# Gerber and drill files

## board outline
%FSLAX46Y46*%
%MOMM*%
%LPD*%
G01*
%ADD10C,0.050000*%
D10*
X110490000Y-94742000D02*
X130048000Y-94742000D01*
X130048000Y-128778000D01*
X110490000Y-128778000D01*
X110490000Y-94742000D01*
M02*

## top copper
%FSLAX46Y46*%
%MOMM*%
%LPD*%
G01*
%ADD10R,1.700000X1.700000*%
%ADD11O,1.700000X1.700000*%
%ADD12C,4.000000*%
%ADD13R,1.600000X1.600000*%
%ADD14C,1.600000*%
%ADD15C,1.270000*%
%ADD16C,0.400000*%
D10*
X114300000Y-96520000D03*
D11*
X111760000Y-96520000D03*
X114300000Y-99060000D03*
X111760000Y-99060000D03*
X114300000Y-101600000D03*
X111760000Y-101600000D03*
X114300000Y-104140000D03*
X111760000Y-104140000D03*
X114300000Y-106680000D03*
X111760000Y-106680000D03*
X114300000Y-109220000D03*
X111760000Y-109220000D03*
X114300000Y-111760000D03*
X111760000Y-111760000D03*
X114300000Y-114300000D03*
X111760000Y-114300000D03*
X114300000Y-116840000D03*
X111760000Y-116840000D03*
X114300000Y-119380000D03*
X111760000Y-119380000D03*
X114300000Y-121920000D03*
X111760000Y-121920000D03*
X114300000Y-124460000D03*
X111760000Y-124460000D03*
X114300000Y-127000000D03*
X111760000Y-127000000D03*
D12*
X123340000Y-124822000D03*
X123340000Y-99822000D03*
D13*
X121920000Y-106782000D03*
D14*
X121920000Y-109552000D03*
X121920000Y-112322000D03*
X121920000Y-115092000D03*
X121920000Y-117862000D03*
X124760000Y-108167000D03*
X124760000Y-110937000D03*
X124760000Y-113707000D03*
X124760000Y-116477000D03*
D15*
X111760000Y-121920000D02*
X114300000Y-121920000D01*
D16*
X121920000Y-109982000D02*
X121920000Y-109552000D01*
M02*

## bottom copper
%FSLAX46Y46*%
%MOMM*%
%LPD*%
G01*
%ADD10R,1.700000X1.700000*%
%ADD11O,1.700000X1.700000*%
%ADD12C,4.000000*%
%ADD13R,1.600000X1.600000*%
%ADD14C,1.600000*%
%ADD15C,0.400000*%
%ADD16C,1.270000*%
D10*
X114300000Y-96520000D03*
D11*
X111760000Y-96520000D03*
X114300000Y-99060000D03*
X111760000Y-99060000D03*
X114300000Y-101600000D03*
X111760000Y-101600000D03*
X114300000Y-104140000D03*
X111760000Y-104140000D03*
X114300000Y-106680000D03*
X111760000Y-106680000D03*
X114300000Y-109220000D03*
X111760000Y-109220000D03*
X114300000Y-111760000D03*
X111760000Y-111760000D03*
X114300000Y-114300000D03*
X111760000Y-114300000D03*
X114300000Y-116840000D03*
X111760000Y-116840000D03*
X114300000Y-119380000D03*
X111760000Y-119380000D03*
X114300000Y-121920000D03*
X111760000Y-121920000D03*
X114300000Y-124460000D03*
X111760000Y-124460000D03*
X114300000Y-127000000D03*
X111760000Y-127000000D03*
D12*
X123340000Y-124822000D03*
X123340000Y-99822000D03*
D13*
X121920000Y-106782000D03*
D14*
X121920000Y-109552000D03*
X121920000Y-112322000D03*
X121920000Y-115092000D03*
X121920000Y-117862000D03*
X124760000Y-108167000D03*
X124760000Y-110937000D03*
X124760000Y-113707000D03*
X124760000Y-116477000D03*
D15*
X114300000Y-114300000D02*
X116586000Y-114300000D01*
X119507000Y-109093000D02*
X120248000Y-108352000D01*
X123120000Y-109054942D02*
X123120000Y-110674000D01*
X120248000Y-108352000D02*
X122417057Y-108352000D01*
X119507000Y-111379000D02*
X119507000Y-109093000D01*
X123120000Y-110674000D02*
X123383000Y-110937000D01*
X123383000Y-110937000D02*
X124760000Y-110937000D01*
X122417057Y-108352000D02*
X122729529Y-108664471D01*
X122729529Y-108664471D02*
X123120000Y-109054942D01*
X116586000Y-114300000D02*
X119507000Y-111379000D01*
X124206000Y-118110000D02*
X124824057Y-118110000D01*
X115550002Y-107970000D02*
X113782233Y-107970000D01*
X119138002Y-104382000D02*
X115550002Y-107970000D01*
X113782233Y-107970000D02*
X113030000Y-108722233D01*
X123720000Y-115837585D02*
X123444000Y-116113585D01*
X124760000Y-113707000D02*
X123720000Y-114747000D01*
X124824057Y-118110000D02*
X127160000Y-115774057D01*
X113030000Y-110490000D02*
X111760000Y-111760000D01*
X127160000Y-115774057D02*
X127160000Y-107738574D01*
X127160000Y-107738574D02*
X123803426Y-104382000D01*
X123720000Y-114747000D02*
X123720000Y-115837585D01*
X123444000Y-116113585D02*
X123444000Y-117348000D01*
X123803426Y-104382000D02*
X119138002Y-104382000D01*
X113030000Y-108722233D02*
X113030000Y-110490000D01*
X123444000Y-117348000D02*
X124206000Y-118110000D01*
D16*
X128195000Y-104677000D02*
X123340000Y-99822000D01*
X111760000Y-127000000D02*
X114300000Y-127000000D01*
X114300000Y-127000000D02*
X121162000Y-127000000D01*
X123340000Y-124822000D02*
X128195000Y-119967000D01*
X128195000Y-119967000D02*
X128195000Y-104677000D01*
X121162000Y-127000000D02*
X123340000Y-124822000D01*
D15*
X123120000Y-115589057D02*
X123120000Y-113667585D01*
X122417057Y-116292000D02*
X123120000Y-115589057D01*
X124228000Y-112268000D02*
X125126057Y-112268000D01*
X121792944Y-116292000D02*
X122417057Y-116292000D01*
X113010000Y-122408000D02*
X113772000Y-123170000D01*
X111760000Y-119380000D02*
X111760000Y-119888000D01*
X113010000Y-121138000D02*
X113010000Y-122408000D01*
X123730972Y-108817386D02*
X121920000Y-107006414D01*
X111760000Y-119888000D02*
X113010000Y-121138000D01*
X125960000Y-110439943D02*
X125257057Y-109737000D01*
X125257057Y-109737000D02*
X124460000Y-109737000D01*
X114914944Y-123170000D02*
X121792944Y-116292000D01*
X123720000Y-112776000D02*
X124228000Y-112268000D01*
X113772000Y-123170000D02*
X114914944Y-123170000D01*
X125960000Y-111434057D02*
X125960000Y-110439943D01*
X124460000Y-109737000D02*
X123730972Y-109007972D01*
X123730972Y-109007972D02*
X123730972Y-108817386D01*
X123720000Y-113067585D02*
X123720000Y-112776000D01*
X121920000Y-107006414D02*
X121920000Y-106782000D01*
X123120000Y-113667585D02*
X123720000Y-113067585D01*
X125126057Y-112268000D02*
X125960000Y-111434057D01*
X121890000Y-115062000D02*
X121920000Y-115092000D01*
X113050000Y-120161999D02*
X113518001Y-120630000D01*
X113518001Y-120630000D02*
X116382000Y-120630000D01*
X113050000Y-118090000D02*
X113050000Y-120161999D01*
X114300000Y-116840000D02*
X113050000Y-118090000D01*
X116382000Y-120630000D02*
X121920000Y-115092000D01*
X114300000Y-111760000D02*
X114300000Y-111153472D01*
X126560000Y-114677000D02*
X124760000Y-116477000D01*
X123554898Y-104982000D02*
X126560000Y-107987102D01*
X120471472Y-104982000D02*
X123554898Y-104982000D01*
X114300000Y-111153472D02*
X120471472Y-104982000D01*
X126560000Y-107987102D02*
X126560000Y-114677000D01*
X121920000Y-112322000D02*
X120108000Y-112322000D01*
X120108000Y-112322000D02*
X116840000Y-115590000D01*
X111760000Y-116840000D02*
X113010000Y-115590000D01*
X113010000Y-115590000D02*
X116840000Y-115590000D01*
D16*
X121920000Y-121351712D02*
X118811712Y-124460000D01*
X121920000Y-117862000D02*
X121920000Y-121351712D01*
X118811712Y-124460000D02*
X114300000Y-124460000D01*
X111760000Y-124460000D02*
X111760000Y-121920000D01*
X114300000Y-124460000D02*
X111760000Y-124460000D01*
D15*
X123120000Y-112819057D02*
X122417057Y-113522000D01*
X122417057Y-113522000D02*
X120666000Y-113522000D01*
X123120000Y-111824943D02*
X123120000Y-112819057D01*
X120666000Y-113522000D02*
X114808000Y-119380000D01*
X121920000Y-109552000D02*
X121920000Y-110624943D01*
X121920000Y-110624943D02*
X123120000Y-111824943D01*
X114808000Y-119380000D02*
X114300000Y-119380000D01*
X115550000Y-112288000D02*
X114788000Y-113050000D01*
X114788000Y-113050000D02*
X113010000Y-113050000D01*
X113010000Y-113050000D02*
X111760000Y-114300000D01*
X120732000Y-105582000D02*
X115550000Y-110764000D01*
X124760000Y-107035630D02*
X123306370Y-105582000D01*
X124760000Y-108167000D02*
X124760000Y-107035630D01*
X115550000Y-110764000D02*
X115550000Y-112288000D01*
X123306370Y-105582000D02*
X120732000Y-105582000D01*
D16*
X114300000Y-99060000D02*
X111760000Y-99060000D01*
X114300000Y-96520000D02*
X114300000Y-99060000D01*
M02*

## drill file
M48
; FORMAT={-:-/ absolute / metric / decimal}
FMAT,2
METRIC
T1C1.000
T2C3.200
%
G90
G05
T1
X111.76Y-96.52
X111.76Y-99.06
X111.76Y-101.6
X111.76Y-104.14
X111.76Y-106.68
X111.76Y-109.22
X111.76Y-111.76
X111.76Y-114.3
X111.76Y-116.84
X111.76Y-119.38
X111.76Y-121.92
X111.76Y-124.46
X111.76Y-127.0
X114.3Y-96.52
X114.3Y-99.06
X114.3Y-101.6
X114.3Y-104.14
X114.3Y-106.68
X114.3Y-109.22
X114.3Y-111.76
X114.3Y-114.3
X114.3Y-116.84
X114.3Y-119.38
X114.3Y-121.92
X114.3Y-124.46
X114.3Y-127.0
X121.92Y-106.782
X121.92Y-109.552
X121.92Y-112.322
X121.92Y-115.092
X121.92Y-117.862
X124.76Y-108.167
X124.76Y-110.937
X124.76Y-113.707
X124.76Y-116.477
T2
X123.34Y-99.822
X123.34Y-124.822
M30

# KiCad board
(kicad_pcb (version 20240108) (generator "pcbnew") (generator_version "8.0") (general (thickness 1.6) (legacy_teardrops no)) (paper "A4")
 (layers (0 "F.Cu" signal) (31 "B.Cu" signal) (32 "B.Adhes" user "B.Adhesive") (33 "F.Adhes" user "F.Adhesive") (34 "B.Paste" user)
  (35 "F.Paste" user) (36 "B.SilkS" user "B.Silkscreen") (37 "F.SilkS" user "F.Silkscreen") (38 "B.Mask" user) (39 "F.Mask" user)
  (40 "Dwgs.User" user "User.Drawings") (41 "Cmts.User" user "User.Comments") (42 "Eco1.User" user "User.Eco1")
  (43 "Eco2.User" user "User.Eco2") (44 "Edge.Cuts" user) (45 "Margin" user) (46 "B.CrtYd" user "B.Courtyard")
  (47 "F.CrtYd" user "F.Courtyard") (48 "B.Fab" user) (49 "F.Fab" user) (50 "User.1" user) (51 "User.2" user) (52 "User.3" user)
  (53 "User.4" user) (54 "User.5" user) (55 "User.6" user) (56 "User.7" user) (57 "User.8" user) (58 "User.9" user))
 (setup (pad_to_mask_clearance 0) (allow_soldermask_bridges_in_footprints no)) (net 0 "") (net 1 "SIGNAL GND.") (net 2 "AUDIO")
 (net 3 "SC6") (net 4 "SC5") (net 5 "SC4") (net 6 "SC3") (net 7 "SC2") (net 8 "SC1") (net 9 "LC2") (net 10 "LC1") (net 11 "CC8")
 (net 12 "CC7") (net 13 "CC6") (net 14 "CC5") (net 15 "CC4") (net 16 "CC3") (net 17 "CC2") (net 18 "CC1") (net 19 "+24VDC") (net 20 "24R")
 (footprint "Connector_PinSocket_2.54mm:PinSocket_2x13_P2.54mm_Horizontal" (layer "F.Cu") (at 114.3 96.52)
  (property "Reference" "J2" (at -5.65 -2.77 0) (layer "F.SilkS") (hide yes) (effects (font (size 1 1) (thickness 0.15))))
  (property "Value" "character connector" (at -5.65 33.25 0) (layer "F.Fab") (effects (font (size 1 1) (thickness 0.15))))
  (pad "1" thru_hole rect (at 0 0) (size 1.7 1.7) (drill 1) (layers "*.Cu" "*.Mask") (remove_unused_layers no) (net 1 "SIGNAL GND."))
  (pad "2" thru_hole oval (at -2.54 0) (size 1.7 1.7) (drill 1) (layers "*.Cu" "*.Mask") (remove_unused_layers no) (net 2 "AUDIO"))
  (pad "3" thru_hole oval (at 0 2.54) (size 1.7 1.7) (drill 1) (layers "*.Cu" "*.Mask") (remove_unused_layers no) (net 1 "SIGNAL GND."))
  (pad "4" thru_hole oval (at -2.54 2.54) (size 1.7 1.7) (drill 1) (layers "*.Cu" "*.Mask") (remove_unused_layers no) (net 1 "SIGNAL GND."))
  (pad "5" thru_hole oval (at 0 5.08) (size 1.7 1.7) (drill 1) (layers "*.Cu" "*.Mask") (remove_unused_layers no) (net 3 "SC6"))
  (pad "6" thru_hole oval (at -2.54 5.08) (size 1.7 1.7) (drill 1) (layers "*.Cu" "*.Mask") (remove_unused_layers no) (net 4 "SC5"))
  (pad "7" thru_hole oval (at 0 7.62) (size 1.7 1.7) (drill 1) (layers "*.Cu" "*.Mask") (remove_unused_layers no) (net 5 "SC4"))
  (pad "8" thru_hole oval (at -2.54 7.62) (size 1.7 1.7) (drill 1) (layers "*.Cu" "*.Mask") (remove_unused_layers no) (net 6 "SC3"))
  (pad "9" thru_hole oval (at 0 10.16) (size 1.7 1.7) (drill 1) (layers "*.Cu" "*.Mask") (remove_unused_layers no) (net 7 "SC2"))
  (pad "10" thru_hole oval (at -2.54 10.16) (size 1.7 1.7) (drill 1) (layers "*.Cu" "*.Mask") (remove_unused_layers no) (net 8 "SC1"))
  (pad "11" thru_hole oval (at 0 12.7) (size 1.7 1.7) (drill 1) (layers "*.Cu" "*.Mask") (remove_unused_layers no) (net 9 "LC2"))
  (pad "12" thru_hole oval (at -2.54 12.7) (size 1.7 1.7) (drill 1) (layers "*.Cu" "*.Mask") (remove_unused_layers no) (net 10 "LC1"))
  (pad "13" thru_hole oval (at 0 15.24) (size 1.7 1.7) (drill 1) (layers "*.Cu" "*.Mask") (remove_unused_layers no) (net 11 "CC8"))
  (pad "14" thru_hole oval (at -2.54 15.24) (size 1.7 1.7) (drill 1) (layers "*.Cu" "*.Mask") (remove_unused_layers no) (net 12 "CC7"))
  (pad "15" thru_hole oval (at 0 17.78) (size 1.7 1.7) (drill 1) (layers "*.Cu" "*.Mask") (remove_unused_layers no) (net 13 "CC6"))
  (pad "16" thru_hole oval (at -2.54 17.78) (size 1.7 1.7) (drill 1) (layers "*.Cu" "*.Mask") (remove_unused_layers no) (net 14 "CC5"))
  (pad "17" thru_hole oval (at 0 20.32) (size 1.7 1.7) (drill 1) (layers "*.Cu" "*.Mask") (remove_unused_layers no) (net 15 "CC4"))
  (pad "18" thru_hole oval (at -2.54 20.32) (size 1.7 1.7) (drill 1) (layers "*.Cu" "*.Mask") (remove_unused_layers no) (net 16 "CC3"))
  (pad "19" thru_hole oval (at 0 22.86) (size 1.7 1.7) (drill 1) (layers "*.Cu" "*.Mask") (remove_unused_layers no) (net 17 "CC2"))
  (pad "20" thru_hole oval (at -2.54 22.86) (size 1.7 1.7) (drill 1) (layers "*.Cu" "*.Mask") (remove_unused_layers no) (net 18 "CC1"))
  (pad "21" thru_hole oval (at 0 25.4) (size 1.7 1.7) (drill 1) (layers "*.Cu" "*.Mask") (remove_unused_layers no) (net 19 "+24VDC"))
  (pad "22" thru_hole oval (at -2.54 25.4) (size 1.7 1.7) (drill 1) (layers "*.Cu" "*.Mask") (remove_unused_layers no) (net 19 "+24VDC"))
  (pad "23" thru_hole oval (at 0 27.94) (size 1.7 1.7) (drill 1) (layers "*.Cu" "*.Mask") (remove_unused_layers no) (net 19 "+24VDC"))
  (pad "24" thru_hole oval (at -2.54 27.94) (size 1.7 1.7) (drill 1) (layers "*.Cu" "*.Mask") (remove_unused_layers no) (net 19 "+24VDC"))
  (pad "25" thru_hole oval (at 0 30.48) (size 1.7 1.7) (drill 1) (layers "*.Cu" "*.Mask") (remove_unused_layers no) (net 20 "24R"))
  (pad "26" thru_hole oval (at -2.54 30.48) (size 1.7 1.7) (drill 1) (layers "*.Cu" "*.Mask") (remove_unused_layers no) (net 20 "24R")))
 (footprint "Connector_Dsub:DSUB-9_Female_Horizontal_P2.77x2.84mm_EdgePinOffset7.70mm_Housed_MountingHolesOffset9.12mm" (layer "F.Cu")
  (at 121.92 106.782 90)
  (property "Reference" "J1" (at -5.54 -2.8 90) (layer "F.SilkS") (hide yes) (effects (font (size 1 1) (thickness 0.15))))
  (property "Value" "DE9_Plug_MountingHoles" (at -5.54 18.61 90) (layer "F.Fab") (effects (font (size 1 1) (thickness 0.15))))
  (pad "0" thru_hole circle (at -18.04 1.42 90) (size 4 4) (drill 3.2) (layers "*.Cu" "*.Mask") (remove_unused_layers no) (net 20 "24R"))
  (pad "0" thru_hole circle (at 6.96 1.42 90) (size 4 4) (drill 3.2) (layers "*.Cu" "*.Mask") (remove_unused_layers no) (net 20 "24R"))
  (pad "1" thru_hole rect (at 0 0 90) (size 1.6 1.6) (drill 1) (layers "*.Cu" "*.Mask") (remove_unused_layers no) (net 18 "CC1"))
  (pad "2" thru_hole circle (at -2.77 0 90) (size 1.6 1.6) (drill 1) (layers "*.Cu" "*.Mask") (remove_unused_layers no) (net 17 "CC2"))
  (pad "3" thru_hole circle (at -5.54 0 90) (size 1.6 1.6) (drill 1) (layers "*.Cu" "*.Mask") (remove_unused_layers no) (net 16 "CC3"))
  (pad "4" thru_hole circle (at -8.31 0 90) (size 1.6 1.6) (drill 1) (layers "*.Cu" "*.Mask") (remove_unused_layers no) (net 15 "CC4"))
  (pad "5" thru_hole circle (at -11.08 0 90) (size 1.6 1.6) (drill 1) (layers "*.Cu" "*.Mask") (remove_unused_layers no) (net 19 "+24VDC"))
  (pad "6" thru_hole circle (at -1.385 2.84 90) (size 1.6 1.6) (drill 1) (layers "*.Cu" "*.Mask") (remove_unused_layers no) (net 14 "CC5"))
  (pad "7" thru_hole circle (at -4.155 2.84 90) (size 1.6 1.6) (drill 1) (layers "*.Cu" "*.Mask") (remove_unused_layers no) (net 13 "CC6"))
  (pad "8" thru_hole circle (at -6.925 2.84 90) (size 1.6 1.6) (drill 1) (layers "*.Cu" "*.Mask") (remove_unused_layers no) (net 12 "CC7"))
  (pad "9" thru_hole circle (at -9.695 2.84 90) (size 1.6 1.6) (drill 1) (layers "*.Cu" "*.Mask") (remove_unused_layers no) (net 11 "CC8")))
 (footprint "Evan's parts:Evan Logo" (layer "B.Cu") (at 127.254 97.536 -90)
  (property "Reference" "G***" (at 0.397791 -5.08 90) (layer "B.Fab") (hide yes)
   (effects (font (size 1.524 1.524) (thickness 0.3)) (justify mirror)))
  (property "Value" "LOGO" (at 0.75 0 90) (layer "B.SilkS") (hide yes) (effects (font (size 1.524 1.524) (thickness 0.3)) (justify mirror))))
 (gr_rect (start 110.49 94.742) (end 130.048 128.778) (stroke (width 0.05) (type default)) (fill none) (layer "Edge.Cuts"))
 (segment (start 114.3 114.3) (end 116.586 114.3) (width 0.4) (layer "B.Cu") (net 13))
 (segment (start 119.507 109.093) (end 120.248 108.352) (width 0.4) (layer "B.Cu") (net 13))
 (segment (start 123.12 109.054942) (end 123.12 110.674) (width 0.4) (layer "B.Cu") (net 13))
 (segment (start 120.248 108.352) (end 122.417057 108.352) (width 0.4) (layer "B.Cu") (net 13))
 (segment (start 119.507 111.379) (end 119.507 109.093) (width 0.4) (layer "B.Cu") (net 13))
 (segment (start 123.12 110.674) (end 123.383 110.937) (width 0.4) (layer "B.Cu") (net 13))
 (segment (start 123.383 110.937) (end 124.76 110.937) (width 0.4) (layer "B.Cu") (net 13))
 (segment (start 122.417057 108.352) (end 122.729529 108.664471) (width 0.4) (layer "B.Cu") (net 13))
 (segment (start 122.729529 108.664471) (end 123.12 109.054942) (width 0.4) (layer "B.Cu") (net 13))
 (segment (start 116.586 114.3) (end 119.507 111.379) (width 0.4) (layer "B.Cu") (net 13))
 (segment (start 124.206 118.11) (end 124.824057 118.11) (width 0.4) (layer "B.Cu") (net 12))
 (segment (start 115.550002 107.97) (end 113.782233 107.97) (width 0.4) (layer "B.Cu") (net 12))
 (segment (start 119.138002 104.382) (end 115.550002 107.97) (width 0.4) (layer "B.Cu") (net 12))
 (segment (start 113.782233 107.97) (end 113.03 108.722233) (width 0.4) (layer "B.Cu") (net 12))
 (segment (start 123.72 115.837585) (end 123.444 116.113585) (width 0.4) (layer "B.Cu") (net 12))
 (segment (start 124.76 113.707) (end 123.72 114.747) (width 0.4) (layer "B.Cu") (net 12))
 (segment (start 124.824057 118.11) (end 127.16 115.774057) (width 0.4) (layer "B.Cu") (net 12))
 (segment (start 113.03 110.49) (end 111.76 111.76) (width 0.4) (layer "B.Cu") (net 12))
 (segment (start 127.16 115.774057) (end 127.16 107.738574) (width 0.4) (layer "B.Cu") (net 12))
 (segment (start 127.16 107.738574) (end 123.803426 104.382) (width 0.4) (layer "B.Cu") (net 12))
 (segment (start 123.72 114.747) (end 123.72 115.837585) (width 0.4) (layer "B.Cu") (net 12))
 (segment (start 123.444 116.113585) (end 123.444 117.348) (width 0.4) (layer "B.Cu") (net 12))
 (segment (start 123.803426 104.382) (end 119.138002 104.382) (width 0.4) (layer "B.Cu") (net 12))
 (segment (start 113.03 108.722233) (end 113.03 110.49) (width 0.4) (layer "B.Cu") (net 12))
 (segment (start 123.444 117.348) (end 124.206 118.11) (width 0.4) (layer "B.Cu") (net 12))
 (segment (start 128.195 104.677) (end 123.34 99.822) (width 1.27) (layer "B.Cu") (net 20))
 (segment (start 111.76 127) (end 114.3 127) (width 1.27) (layer "B.Cu") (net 20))
 (segment (start 114.3 127) (end 121.162 127) (width 1.27) (layer "B.Cu") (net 20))
 (segment (start 123.34 124.822) (end 128.195 119.967) (width 1.27) (layer "B.Cu") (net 20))
 (segment (start 128.195 119.967) (end 128.195 104.677) (width 1.27) (layer "B.Cu") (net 20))
 (segment (start 121.162 127) (end 123.34 124.822) (width 1.27) (layer "B.Cu") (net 20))
 (segment (start 123.12 115.589057) (end 123.12 113.667585) (width 0.4) (layer "B.Cu") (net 18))
 (segment (start 122.417057 116.292) (end 123.12 115.589057) (width 0.4) (layer "B.Cu") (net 18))
 (segment (start 124.228 112.268) (end 125.126057 112.268) (width 0.4) (layer "B.Cu") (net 18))
 (segment (start 121.792944 116.292) (end 122.417057 116.292) (width 0.4) (layer "B.Cu") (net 18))
 (segment (start 113.01 122.408) (end 113.772 123.17) (width 0.4) (layer "B.Cu") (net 18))
 (segment (start 111.76 119.38) (end 111.76 119.888) (width 0.4) (layer "B.Cu") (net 18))
 (segment (start 113.01 121.138) (end 113.01 122.408) (width 0.4) (layer "B.Cu") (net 18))
 (segment (start 123.730972 108.817386) (end 121.92 107.006414) (width 0.4) (layer "B.Cu") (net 18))
 (segment (start 111.76 119.888) (end 113.01 121.138) (width 0.4) (layer "B.Cu") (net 18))
 (segment (start 125.96 110.439943) (end 125.257057 109.737) (width 0.4) (layer "B.Cu") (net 18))
 (segment (start 125.257057 109.737) (end 124.46 109.737) (width 0.4) (layer "B.Cu") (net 18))
 (segment (start 114.914944 123.17) (end 121.792944 116.292) (width 0.4) (layer "B.Cu") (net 18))
 (segment (start 123.72 112.776) (end 124.228 112.268) (width 0.4) (layer "B.Cu") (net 18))
 (segment (start 113.772 123.17) (end 114.914944 123.17) (width 0.4) (layer "B.Cu") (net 18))
 (segment (start 125.96 111.434057) (end 125.96 110.439943) (width 0.4) (layer "B.Cu") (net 18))
 (segment (start 124.46 109.737) (end 123.730972 109.007972) (width 0.4) (layer "B.Cu") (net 18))
 (segment (start 123.730972 109.007972) (end 123.730972 108.817386) (width 0.4) (layer "B.Cu") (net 18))
 (segment (start 123.72 113.067585) (end 123.72 112.776) (width 0.4) (layer "B.Cu") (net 18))
 (segment (start 121.92 107.006414) (end 121.92 106.782) (width 0.4) (layer "B.Cu") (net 18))
 (segment (start 123.12 113.667585) (end 123.72 113.067585) (width 0.4) (layer "B.Cu") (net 18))
 (segment (start 125.126057 112.268) (end 125.96 111.434057) (width 0.4) (layer "B.Cu") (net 18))
 (segment (start 121.89 115.062) (end 121.92 115.092) (width 0.4) (layer "B.Cu") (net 15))
 (segment (start 113.05 120.161999) (end 113.518001 120.63) (width 0.4) (layer "B.Cu") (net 15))
 (segment (start 113.518001 120.63) (end 116.382 120.63) (width 0.4) (layer "B.Cu") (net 15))
 (segment (start 113.05 118.09) (end 113.05 120.161999) (width 0.4) (layer "B.Cu") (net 15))
 (segment (start 114.3 116.84) (end 113.05 118.09) (width 0.4) (layer "B.Cu") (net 15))
 (segment (start 116.382 120.63) (end 121.92 115.092) (width 0.4) (layer "B.Cu") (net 15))
 (segment (start 114.3 111.76) (end 114.3 111.153472) (width 0.4) (layer "B.Cu") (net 11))
 (segment (start 126.56 114.677) (end 124.76 116.477) (width 0.4) (layer "B.Cu") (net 11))
 (segment (start 123.554898 104.982) (end 126.56 107.987102) (width 0.4) (layer "B.Cu") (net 11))
 (segment (start 120.471472 104.982) (end 123.554898 104.982) (width 0.4) (layer "B.Cu") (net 11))
 (segment (start 114.3 111.153472) (end 120.471472 104.982) (width 0.4) (layer "B.Cu") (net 11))
 (segment (start 126.56 107.987102) (end 126.56 114.677) (width 0.4) (layer "B.Cu") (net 11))
 (segment (start 121.92 112.322) (end 120.108 112.322) (width 0.4) (layer "B.Cu") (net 16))
 (segment (start 120.108 112.322) (end 116.84 115.59) (width 0.4) (layer "B.Cu") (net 16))
 (segment (start 111.76 116.84) (end 113.01 115.59) (width 0.4) (layer "B.Cu") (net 16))
 (segment (start 113.01 115.59) (end 116.84 115.59) (width 0.4) (layer "B.Cu") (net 16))
 (segment (start 111.76 121.92) (end 114.3 121.92) (width 1.27) (layer "F.Cu") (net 19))
 (segment (start 121.92 121.351712) (end 118.811712 124.46) (width 1.27) (layer "B.Cu") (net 19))
 (segment (start 121.92 117.862) (end 121.92 121.351712) (width 1.27) (layer "B.Cu") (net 19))
 (segment (start 118.811712 124.46) (end 114.3 124.46) (width 1.27) (layer "B.Cu") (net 19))
 (segment (start 111.76 124.46) (end 111.76 121.92) (width 1.27) (layer "B.Cu") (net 19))
 (segment (start 114.3 124.46) (end 111.76 124.46) (width 1.27) (layer "B.Cu") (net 19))
 (segment (start 121.92 109.982) (end 121.92 109.552) (width 0.4) (layer "F.Cu") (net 17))
 (segment (start 123.12 112.819057) (end 122.417057 113.522) (width 0.4) (layer "B.Cu") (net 17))
 (segment (start 122.417057 113.522) (end 120.666 113.522) (width 0.4) (layer "B.Cu") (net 17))
 (segment (start 123.12 111.824943) (end 123.12 112.819057) (width 0.4) (layer "B.Cu") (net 17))
 (segment (start 120.666 113.522) (end 114.808 119.38) (width 0.4) (layer "B.Cu") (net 17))
 (segment (start 121.92 109.552) (end 121.92 110.624943) (width 0.4) (layer "B.Cu") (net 17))
 (segment (start 121.92 110.624943) (end 123.12 111.824943) (width 0.4) (layer "B.Cu") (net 17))
 (segment (start 114.808 119.38) (end 114.3 119.38) (width 0.4) (layer "B.Cu") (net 17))
 (segment (start 115.55 112.288) (end 114.788 113.05) (width 0.4) (layer "B.Cu") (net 14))
 (segment (start 114.788 113.05) (end 113.01 113.05) (width 0.4) (layer "B.Cu") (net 14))
 (segment (start 113.01 113.05) (end 111.76 114.3) (width 0.4) (layer "B.Cu") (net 14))
 (segment (start 120.732 105.582) (end 115.55 110.764) (width 0.4) (layer "B.Cu") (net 14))
 (segment (start 124.76 107.03563) (end 123.30637 105.582) (width 0.4) (layer "B.Cu") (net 14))
 (segment (start 124.76 108.167) (end 124.76 107.03563) (width 0.4) (layer "B.Cu") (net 14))
 (segment (start 115.55 110.764) (end 115.55 112.288) (width 0.4) (layer "B.Cu") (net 14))
 (segment (start 123.30637 105.582) (end 120.732 105.582) (width 0.4) (layer "B.Cu") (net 14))
 (segment (start 114.3 99.06) (end 111.76 99.06) (width 1.27) (layer "B.Cu") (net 1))
 (segment (start 114.3 96.52) (end 114.3 99.06) (width 1.27) (layer "B.Cu") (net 1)))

